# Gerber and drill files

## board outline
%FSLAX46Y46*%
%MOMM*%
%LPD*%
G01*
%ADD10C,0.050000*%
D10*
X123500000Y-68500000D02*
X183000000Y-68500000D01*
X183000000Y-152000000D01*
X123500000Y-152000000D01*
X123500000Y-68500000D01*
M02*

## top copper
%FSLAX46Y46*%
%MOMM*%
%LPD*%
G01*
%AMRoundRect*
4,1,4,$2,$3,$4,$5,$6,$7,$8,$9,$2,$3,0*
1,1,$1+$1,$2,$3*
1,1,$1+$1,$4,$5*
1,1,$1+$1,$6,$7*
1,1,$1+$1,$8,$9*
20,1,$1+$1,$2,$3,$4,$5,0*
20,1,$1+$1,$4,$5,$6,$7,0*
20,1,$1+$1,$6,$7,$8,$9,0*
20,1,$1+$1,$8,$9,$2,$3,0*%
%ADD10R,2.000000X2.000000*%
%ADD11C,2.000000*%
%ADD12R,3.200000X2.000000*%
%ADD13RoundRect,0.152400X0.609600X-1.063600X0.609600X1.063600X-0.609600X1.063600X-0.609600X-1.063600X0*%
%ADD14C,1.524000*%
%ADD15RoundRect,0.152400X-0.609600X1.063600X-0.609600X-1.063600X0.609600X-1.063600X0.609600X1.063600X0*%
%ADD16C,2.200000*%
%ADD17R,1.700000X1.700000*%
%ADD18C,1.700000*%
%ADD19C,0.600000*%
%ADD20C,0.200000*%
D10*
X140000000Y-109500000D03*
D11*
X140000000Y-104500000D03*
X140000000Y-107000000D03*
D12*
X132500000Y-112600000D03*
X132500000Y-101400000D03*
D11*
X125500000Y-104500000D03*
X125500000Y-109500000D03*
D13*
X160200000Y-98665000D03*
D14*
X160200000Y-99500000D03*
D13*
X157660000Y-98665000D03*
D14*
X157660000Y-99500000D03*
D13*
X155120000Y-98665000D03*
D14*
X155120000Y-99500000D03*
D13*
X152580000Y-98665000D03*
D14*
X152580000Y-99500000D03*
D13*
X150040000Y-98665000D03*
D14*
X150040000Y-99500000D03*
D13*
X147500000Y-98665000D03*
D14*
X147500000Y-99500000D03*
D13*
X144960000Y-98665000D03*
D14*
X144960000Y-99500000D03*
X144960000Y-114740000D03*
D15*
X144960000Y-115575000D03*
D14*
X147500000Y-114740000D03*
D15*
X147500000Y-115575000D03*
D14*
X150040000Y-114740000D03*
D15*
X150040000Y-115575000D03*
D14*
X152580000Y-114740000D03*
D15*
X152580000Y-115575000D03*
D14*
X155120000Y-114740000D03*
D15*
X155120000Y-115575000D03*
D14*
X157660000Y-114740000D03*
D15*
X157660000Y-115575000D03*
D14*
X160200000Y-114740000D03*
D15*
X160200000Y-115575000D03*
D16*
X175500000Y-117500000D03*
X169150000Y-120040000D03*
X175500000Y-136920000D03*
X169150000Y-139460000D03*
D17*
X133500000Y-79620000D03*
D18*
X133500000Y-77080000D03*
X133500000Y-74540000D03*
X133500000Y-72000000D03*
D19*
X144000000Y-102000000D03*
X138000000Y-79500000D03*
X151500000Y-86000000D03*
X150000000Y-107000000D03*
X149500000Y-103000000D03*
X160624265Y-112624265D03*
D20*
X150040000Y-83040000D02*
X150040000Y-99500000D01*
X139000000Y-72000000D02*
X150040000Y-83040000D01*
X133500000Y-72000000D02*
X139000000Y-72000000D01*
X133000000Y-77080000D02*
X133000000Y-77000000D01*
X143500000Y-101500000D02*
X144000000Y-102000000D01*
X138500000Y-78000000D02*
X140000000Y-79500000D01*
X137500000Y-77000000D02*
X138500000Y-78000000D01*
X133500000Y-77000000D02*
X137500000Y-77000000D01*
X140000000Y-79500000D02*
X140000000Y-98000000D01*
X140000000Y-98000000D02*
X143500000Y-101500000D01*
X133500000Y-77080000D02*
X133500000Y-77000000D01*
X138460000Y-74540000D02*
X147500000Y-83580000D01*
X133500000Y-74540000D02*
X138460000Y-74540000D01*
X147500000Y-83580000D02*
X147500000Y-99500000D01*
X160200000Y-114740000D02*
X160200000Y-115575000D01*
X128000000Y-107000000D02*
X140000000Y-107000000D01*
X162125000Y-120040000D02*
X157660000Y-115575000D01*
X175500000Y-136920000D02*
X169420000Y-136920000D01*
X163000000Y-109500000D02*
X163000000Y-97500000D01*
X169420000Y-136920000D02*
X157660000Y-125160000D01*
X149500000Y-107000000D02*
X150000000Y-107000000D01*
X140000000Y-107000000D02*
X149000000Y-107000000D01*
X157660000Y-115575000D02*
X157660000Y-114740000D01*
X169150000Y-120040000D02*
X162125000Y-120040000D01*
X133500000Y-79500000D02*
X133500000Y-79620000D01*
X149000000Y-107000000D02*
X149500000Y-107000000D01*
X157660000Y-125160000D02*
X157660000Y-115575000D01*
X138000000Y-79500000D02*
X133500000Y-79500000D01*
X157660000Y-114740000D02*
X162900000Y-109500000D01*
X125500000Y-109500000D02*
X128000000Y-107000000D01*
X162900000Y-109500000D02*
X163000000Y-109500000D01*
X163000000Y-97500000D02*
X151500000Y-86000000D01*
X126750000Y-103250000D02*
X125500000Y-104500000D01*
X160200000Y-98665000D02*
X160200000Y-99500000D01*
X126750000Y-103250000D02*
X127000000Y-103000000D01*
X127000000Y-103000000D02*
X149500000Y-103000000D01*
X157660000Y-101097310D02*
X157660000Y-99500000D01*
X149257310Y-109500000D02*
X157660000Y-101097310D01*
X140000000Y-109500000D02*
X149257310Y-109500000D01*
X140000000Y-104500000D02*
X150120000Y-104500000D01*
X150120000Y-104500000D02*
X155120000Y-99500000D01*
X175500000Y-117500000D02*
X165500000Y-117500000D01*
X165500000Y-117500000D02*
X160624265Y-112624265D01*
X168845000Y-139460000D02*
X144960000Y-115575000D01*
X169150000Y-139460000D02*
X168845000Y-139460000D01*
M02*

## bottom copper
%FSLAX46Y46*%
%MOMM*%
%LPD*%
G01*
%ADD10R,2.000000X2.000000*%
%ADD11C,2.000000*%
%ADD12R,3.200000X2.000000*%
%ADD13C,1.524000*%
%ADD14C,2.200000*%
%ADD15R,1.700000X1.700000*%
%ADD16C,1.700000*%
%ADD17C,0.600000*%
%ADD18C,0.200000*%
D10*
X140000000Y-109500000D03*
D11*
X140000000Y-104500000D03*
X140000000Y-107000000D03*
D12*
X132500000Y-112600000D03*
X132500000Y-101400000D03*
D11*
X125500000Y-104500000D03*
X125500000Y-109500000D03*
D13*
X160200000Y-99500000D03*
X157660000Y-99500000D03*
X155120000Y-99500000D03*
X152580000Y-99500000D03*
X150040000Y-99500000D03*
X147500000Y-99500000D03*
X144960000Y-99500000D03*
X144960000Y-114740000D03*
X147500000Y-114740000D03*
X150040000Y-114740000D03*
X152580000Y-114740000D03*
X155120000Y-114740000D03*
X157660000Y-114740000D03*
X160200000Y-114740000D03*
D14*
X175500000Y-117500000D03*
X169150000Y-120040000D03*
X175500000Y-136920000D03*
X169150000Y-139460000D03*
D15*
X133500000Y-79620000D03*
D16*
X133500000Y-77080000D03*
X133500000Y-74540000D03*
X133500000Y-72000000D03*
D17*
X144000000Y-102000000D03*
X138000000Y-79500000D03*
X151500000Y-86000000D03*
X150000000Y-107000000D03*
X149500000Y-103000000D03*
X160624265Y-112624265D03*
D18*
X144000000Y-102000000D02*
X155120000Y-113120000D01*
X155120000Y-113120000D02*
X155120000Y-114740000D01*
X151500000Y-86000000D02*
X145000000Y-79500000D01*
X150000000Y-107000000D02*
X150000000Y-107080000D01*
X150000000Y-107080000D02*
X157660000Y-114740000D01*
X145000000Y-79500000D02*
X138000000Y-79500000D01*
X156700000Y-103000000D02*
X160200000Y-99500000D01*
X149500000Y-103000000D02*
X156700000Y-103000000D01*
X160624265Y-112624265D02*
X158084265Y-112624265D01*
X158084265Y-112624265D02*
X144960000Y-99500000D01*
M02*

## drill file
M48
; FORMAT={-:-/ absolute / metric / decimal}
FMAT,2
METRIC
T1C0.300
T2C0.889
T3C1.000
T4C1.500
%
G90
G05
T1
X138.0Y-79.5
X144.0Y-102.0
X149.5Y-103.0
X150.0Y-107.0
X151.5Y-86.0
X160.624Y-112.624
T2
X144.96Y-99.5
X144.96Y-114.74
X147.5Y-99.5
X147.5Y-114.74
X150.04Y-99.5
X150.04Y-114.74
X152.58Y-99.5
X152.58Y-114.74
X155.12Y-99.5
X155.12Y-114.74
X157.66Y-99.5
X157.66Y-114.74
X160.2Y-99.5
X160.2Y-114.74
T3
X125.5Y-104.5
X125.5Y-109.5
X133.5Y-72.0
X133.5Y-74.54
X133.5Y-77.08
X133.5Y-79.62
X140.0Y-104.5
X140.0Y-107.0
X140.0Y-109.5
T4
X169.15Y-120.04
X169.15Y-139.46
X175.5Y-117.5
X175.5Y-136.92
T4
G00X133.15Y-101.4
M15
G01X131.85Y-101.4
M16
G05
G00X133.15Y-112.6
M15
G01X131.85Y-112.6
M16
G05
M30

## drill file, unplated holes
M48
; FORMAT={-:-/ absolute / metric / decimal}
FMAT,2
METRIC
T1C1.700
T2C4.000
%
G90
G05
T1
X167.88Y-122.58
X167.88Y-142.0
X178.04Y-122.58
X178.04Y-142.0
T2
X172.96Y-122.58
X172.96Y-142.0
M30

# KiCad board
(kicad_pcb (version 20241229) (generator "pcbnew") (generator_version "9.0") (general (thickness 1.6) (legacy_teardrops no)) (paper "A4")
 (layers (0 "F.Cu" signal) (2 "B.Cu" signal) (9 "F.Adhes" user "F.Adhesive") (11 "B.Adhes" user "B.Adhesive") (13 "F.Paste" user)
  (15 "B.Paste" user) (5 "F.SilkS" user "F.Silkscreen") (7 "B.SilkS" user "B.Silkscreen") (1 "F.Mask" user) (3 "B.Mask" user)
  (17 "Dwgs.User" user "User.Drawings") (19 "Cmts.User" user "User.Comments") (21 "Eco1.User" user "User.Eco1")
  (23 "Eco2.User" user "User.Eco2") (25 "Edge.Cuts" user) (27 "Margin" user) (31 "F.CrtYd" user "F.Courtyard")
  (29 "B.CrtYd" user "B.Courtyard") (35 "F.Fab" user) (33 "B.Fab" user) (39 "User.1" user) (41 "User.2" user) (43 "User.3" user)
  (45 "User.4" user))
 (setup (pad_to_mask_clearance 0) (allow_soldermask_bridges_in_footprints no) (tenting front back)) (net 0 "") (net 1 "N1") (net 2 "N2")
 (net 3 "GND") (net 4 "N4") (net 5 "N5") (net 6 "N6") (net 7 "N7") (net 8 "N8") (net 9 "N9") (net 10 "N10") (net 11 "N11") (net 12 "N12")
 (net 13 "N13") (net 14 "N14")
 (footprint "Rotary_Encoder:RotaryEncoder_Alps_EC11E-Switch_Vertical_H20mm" (layer "F.Cu") (at 140 109.5 180)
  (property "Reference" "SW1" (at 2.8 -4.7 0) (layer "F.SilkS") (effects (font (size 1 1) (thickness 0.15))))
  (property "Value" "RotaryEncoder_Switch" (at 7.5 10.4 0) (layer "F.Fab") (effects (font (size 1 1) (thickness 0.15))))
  (pad "A" thru_hole rect (at 0 0 180) (size 2 2) (drill 1) (layers "*.Cu" "*.Mask") (remove_unused_layers no) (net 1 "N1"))
  (pad "B" thru_hole circle (at 0 5 180) (size 2 2) (drill 1) (layers "*.Cu" "*.Mask") (remove_unused_layers no) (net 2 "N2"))
  (pad "C" thru_hole circle (at 0 2.5 180) (size 2 2) (drill 1) (layers "*.Cu" "*.Mask") (remove_unused_layers no) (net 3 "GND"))
  (pad "MP" thru_hole rect (at 7.5 -3.1 180) (size 3.2 2) (drill oval 2.8 1.5) (layers "*.Cu" "*.Mask") (remove_unused_layers no))
  (pad "MP" thru_hole rect (at 7.5 8.1 180) (size 3.2 2) (drill oval 2.8 1.5) (layers "*.Cu" "*.Mask") (remove_unused_layers no))
  (pad "S1" thru_hole circle (at 14.5 5 180) (size 2 2) (drill 1) (layers "*.Cu" "*.Mask") (remove_unused_layers no) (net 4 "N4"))
  (pad "S2" thru_hole circle (at 14.5 0 180) (size 2 2) (drill 1) (layers "*.Cu" "*.Mask") (remove_unused_layers no) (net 3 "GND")))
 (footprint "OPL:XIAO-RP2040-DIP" (layer "F.Cu") (at 152.58 107.12 -90)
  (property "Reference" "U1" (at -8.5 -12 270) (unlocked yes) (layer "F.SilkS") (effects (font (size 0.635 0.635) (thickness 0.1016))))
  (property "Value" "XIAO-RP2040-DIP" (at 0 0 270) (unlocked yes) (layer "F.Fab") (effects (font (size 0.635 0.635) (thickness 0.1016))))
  (pad "1" smd roundrect (at -8.455 -7.62 90) (size 2.432 1.524) (layers "F.Cu" "F.Mask") (roundrect_rratio 0.1) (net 4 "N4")
   (thermal_bridge_angle 45))
  (pad "1" thru_hole circle (at -7.62 -7.62 90) (size 1.524 1.524) (drill 0.889) (layers "*.Cu" "*.Mask") (remove_unused_layers no)
   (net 4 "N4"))
  (pad "2" smd roundrect (at -8.455 -5.08 90) (size 2.432 1.524) (layers "F.Cu" "F.Mask") (roundrect_rratio 0.1) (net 1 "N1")
   (thermal_bridge_angle 45))
  (pad "2" thru_hole circle (at -7.62 -5.08 90) (size 1.524 1.524) (drill 0.889) (layers "*.Cu" "*.Mask") (remove_unused_layers no)
   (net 1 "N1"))
  (pad "3" smd roundrect (at -8.455 -2.54 90) (size 2.432 1.524) (layers "F.Cu" "F.Mask") (roundrect_rratio 0.1) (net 2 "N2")
   (thermal_bridge_angle 45))
  (pad "3" thru_hole circle (at -7.62 -2.54 90) (size 1.524 1.524) (drill 0.889) (layers "*.Cu" "*.Mask") (remove_unused_layers no)
   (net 2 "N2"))
  (pad "4" smd roundrect (at -8.455 0 90) (size 2.432 1.524) (layers "F.Cu" "F.Mask") (roundrect_rratio 0.1) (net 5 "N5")
   (thermal_bridge_angle 45))
  (pad "4" thru_hole circle (at -7.62 0 90) (size 1.524 1.524) (drill 0.889) (layers "*.Cu" "*.Mask") (remove_unused_layers no) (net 5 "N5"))
  (pad "5" smd roundrect (at -8.455 2.54 90) (size 2.432 1.524) (layers "F.Cu" "F.Mask") (roundrect_rratio 0.1) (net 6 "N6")
   (thermal_bridge_angle 45))
  (pad "5" thru_hole circle (at -7.62 2.54 90) (size 1.524 1.524) (drill 0.889) (layers "*.Cu" "*.Mask") (remove_unused_layers no)
   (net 6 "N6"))
  (pad "6" smd roundrect (at -8.455 5.08 90) (size 2.432 1.524) (layers "F.Cu" "F.Mask") (roundrect_rratio 0.1) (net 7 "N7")
   (thermal_bridge_angle 45))
  (pad "6" thru_hole circle (at -7.62 5.08 90) (size 1.524 1.524) (drill 0.889) (layers "*.Cu" "*.Mask") (remove_unused_layers no)
   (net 7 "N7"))
  (pad "7" smd roundrect (at -8.455 7.62 90) (size 2.432 1.524) (layers "F.Cu" "F.Mask") (roundrect_rratio 0.1) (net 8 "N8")
   (thermal_bridge_angle 45))
  (pad "7" thru_hole circle (at -7.62 7.62 90) (size 1.524 1.524) (drill 0.889) (layers "*.Cu" "*.Mask") (remove_unused_layers no)
   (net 8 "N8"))
  (pad "8" thru_hole circle (at 7.62 7.62 270) (size 1.524 1.524) (drill 0.889) (layers "*.Cu" "*.Mask") (remove_unused_layers no)
   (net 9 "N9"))
  (pad "8" smd roundrect (at 8.455 7.62 270) (size 2.432 1.524) (layers "F.Cu" "F.Mask") (roundrect_rratio 0.1) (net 9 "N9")
   (thermal_bridge_angle 45))
  (pad "9" thru_hole circle (at 7.62 5.08 270) (size 1.524 1.524) (drill 0.889) (layers "*.Cu" "*.Mask") (remove_unused_layers no)
   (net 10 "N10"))
  (pad "9" smd roundrect (at 8.455 5.08 270) (size 2.432 1.524) (layers "F.Cu" "F.Mask") (roundrect_rratio 0.1) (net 10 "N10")
   (thermal_bridge_angle 45))
  (pad "10" thru_hole circle (at 7.62 2.54 270) (size 1.524 1.524) (drill 0.889) (layers "*.Cu" "*.Mask") (remove_unused_layers no)
   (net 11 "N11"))
  (pad "10" smd roundrect (at 8.455 2.54 270) (size 2.432 1.524) (layers "F.Cu" "F.Mask") (roundrect_rratio 0.1) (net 11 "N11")
   (thermal_bridge_angle 45))
  (pad "11" thru_hole circle (at 7.62 0 270) (size 1.524 1.524) (drill 0.889) (layers "*.Cu" "*.Mask") (remove_unused_layers no)
   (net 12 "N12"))
  (pad "11" smd roundrect (at 8.455 0 270) (size 2.432 1.524) (layers "F.Cu" "F.Mask") (roundrect_rratio 0.1) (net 12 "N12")
   (thermal_bridge_angle 45))
  (pad "12" thru_hole circle (at 7.62 -2.54 270) (size 1.524 1.524) (drill 0.889) (layers "*.Cu" "*.Mask") (remove_unused_layers no)
   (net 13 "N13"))
  (pad "12" smd roundrect (at 8.455 -2.54 270) (size 2.432 1.524) (layers "F.Cu" "F.Mask") (roundrect_rratio 0.1) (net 13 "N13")
   (thermal_bridge_angle 45))
  (pad "13" thru_hole circle (at 7.62 -5.08 270) (size 1.524 1.524) (drill 0.889) (layers "*.Cu" "*.Mask") (remove_unused_layers no)
   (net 3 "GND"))
  (pad "13" smd roundrect (at 8.455 -5.08 270) (size 2.432 1.524) (layers "F.Cu" "F.Mask") (roundrect_rratio 0.1) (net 3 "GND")
   (thermal_bridge_angle 45))
  (pad "14" thru_hole circle (at 7.62 -7.62 270) (size 1.524 1.524) (drill 0.889) (layers "*.Cu" "*.Mask") (remove_unused_layers no)
   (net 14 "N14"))
  (pad "14" smd roundrect (at 8.455 -7.62 270) (size 2.432 1.524) (layers "F.Cu" "F.Mask") (roundrect_rratio 0.1) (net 14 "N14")
   (thermal_bridge_angle 45)))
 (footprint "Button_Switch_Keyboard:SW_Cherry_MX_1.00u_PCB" (layer "F.Cu") (at 175.5 117.5)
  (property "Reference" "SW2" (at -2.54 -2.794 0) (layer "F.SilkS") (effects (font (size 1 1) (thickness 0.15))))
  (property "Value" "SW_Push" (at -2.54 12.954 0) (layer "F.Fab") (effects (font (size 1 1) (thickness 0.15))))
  (pad "" np_thru_hole circle (at -7.62 5.08) (size 1.7 1.7) (drill 1.7) (layers "*.Cu" "*.Mask"))
  (pad "" np_thru_hole circle (at -2.54 5.08) (size 4 4) (drill 4) (layers "*.Cu" "*.Mask"))
  (pad "" np_thru_hole circle (at 2.54 5.08) (size 1.7 1.7) (drill 1.7) (layers "*.Cu" "*.Mask"))
  (pad "1" thru_hole circle (at 0 0) (size 2.2 2.2) (drill 1.5) (layers "*.Cu" "*.Mask") (remove_unused_layers no) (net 8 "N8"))
  (pad "2" thru_hole circle (at -6.35 2.54) (size 2.2 2.2) (drill 1.5) (layers "*.Cu" "*.Mask") (remove_unused_layers no) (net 3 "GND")))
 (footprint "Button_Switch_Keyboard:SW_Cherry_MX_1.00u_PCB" (layer "F.Cu") (at 175.5 136.92)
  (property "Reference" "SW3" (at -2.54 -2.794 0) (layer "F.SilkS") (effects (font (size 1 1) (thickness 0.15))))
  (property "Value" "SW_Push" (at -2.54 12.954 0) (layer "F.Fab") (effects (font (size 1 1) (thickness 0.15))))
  (pad "" np_thru_hole circle (at -7.62 5.08) (size 1.7 1.7) (drill 1.7) (layers "*.Cu" "*.Mask"))
  (pad "" np_thru_hole circle (at -2.54 5.08) (size 4 4) (drill 4) (layers "*.Cu" "*.Mask"))
  (pad "" np_thru_hole circle (at 2.54 5.08) (size 1.7 1.7) (drill 1.7) (layers "*.Cu" "*.Mask"))
  (pad "1" thru_hole circle (at 0 0) (size 2.2 2.2) (drill 1.5) (layers "*.Cu" "*.Mask") (remove_unused_layers no) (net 3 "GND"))
  (pad "2" thru_hole circle (at -6.35 2.54) (size 2.2 2.2) (drill 1.5) (layers "*.Cu" "*.Mask") (remove_unused_layers no) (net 9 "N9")))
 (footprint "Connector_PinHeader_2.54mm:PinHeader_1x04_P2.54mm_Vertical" (layer "F.Cu") (at 133.5 79.62 180)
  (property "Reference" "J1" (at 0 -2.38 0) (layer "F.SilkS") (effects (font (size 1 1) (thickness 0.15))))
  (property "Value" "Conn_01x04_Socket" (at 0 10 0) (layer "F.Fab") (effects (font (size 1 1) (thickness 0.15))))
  (pad "1" thru_hole rect (at 0 0 180) (size 1.7 1.7) (drill 1) (layers "*.Cu" "*.Mask") (remove_unused_layers no) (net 3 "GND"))
  (pad "2" thru_hole circle (at 0 2.54 180) (size 1.7 1.7) (drill 1) (layers "*.Cu" "*.Mask") (remove_unused_layers no) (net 13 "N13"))
  (pad "3" thru_hole circle (at 0 5.08 180) (size 1.7 1.7) (drill 1) (layers "*.Cu" "*.Mask") (remove_unused_layers no) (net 7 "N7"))
  (pad "4" thru_hole circle (at 0 7.62 180) (size 1.7 1.7) (drill 1) (layers "*.Cu" "*.Mask") (remove_unused_layers no) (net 6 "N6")))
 (gr_rect (start 123.5 68.5) (end 183 152) (stroke (width 0.05) (type default)) (fill no) (layer "Edge.Cuts"))
 (segment (start 150.04 83.04) (end 150.04 99.5) (width 0.2) (layer "F.Cu") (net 6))
 (segment (start 139 72) (end 150.04 83.04) (width 0.2) (layer "F.Cu") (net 6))
 (segment (start 133.5 72) (end 139 72) (width 0.2) (layer "F.Cu") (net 6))
 (segment (start 133 77.08) (end 133 77) (width 0.2) (layer "F.Cu") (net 13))
 (segment (start 143.5 101.5) (end 144 102) (width 0.2) (layer "F.Cu") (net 13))
 (segment (start 138.5 78) (end 140 79.5) (width 0.2) (layer "F.Cu") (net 13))
 (segment (start 137.5 77) (end 138.5 78) (width 0.2) (layer "F.Cu") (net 13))
 (segment (start 133.5 77) (end 137.5 77) (width 0.2) (layer "F.Cu") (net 13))
 (segment (start 140 79.5) (end 140 98) (width 0.2) (layer "F.Cu") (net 13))
 (segment (start 140 98) (end 143.5 101.5) (width 0.2) (layer "F.Cu") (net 13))
 (segment (start 133.5 77.08) (end 133.5 77) (width 0.2) (layer "F.Cu") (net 13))
 (via (at 144 102) (size 0.6) (drill 0.3) (layers "F.Cu" "B.Cu") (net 13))
 (segment (start 144 102) (end 155.12 113.12) (width 0.2) (layer "B.Cu") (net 13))
 (segment (start 155.12 113.12) (end 155.12 114.74) (width 0.2) (layer "B.Cu") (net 13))
 (segment (start 138.46 74.54) (end 147.5 83.58) (width 0.2) (layer "F.Cu") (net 7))
 (segment (start 133.5 74.54) (end 138.46 74.54) (width 0.2) (layer "F.Cu") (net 7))
 (segment (start 147.5 83.58) (end 147.5 99.5) (width 0.2) (layer "F.Cu") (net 7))
 (segment (start 160.2 114.74) (end 160.2 115.575) (width 0.2) (layer "F.Cu") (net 14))
 (segment (start 128 107) (end 140 107) (width 0.2) (layer "F.Cu") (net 3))
 (segment (start 162.125 120.04) (end 157.66 115.575) (width 0.2) (layer "F.Cu") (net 3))
 (segment (start 175.5 136.92) (end 169.42 136.92) (width 0.2) (layer "F.Cu") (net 3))
 (segment (start 163 109.5) (end 163 97.5) (width 0.2) (layer "F.Cu") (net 3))
 (segment (start 169.42 136.92) (end 157.66 125.16) (width 0.2) (layer "F.Cu") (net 3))
 (segment (start 149.5 107) (end 150 107) (width 0.2) (layer "F.Cu") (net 3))
 (segment (start 140 107) (end 149 107) (width 0.2) (layer "F.Cu") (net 3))
 (segment (start 157.66 115.575) (end 157.66 114.74) (width 0.2) (layer "F.Cu") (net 3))
 (segment (start 169.15 120.04) (end 162.125 120.04) (width 0.2) (layer "F.Cu") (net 3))
 (segment (start 133.5 79.5) (end 133.5 79.62) (width 0.2) (layer "F.Cu") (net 3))
 (segment (start 149 107) (end 149.5 107) (width 0.2) (layer "F.Cu") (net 3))
 (segment (start 157.66 125.16) (end 157.66 115.575) (width 0.2) (layer "F.Cu") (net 3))
 (segment (start 138 79.5) (end 133.5 79.5) (width 0.2) (layer "F.Cu") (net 3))
 (segment (start 157.66 114.74) (end 162.9 109.5) (width 0.2) (layer "F.Cu") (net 3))
 (segment (start 125.5 109.5) (end 128 107) (width 0.2) (layer "F.Cu") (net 3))
 (segment (start 162.9 109.5) (end 163 109.5) (width 0.2) (layer "F.Cu") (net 3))
 (segment (start 163 97.5) (end 151.5 86) (width 0.2) (layer "F.Cu") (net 3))
 (via (at 138 79.5) (size 0.6) (drill 0.3) (layers "F.Cu" "B.Cu") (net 3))
 (via (at 151.5 86) (size 0.6) (drill 0.3) (layers "F.Cu" "B.Cu") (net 3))
 (via (at 150 107) (size 0.6) (drill 0.3) (layers "F.Cu" "B.Cu") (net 3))
 (segment (start 151.5 86) (end 145 79.5) (width 0.2) (layer "B.Cu") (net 3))
 (segment (start 150 107) (end 150 107.08) (width 0.2) (layer "B.Cu") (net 3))
 (segment (start 150 107.08) (end 157.66 114.74) (width 0.2) (layer "B.Cu") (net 3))
 (segment (start 145 79.5) (end 138 79.5) (width 0.2) (layer "B.Cu") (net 3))
 (segment (start 126.75 103.25) (end 125.5 104.5) (width 0.2) (layer "F.Cu") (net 4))
 (segment (start 160.2 98.665) (end 160.2 99.5) (width 0.2) (layer "F.Cu") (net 4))
 (segment (start 126.75 103.25) (end 127 103) (width 0.2) (layer "F.Cu") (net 4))
 (segment (start 127 103) (end 149.5 103) (width 0.2) (layer "F.Cu") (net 4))
 (via (at 149.5 103) (size 0.6) (drill 0.3) (layers "F.Cu" "B.Cu") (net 4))
 (segment (start 156.7 103) (end 160.2 99.5) (width 0.2) (layer "B.Cu") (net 4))
 (segment (start 149.5 103) (end 156.7 103) (width 0.2) (layer "B.Cu") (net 4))
 (segment (start 157.66 101.09731) (end 157.66 99.5) (width 0.2) (layer "F.Cu") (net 1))
 (segment (start 149.25731 109.5) (end 157.66 101.09731) (width 0.2) (layer "F.Cu") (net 1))
 (segment (start 140 109.5) (end 149.25731 109.5) (width 0.2) (layer "F.Cu") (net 1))
 (segment (start 140 104.5) (end 150.12 104.5) (width 0.2) (layer "F.Cu") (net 2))
 (segment (start 150.12 104.5) (end 155.12 99.5) (width 0.2) (layer "F.Cu") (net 2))
 (segment (start 175.5 117.5) (end 165.5 117.5) (width 0.2) (layer "F.Cu") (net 8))
 (segment (start 165.5 117.5) (end 160.624265 112.624265) (width 0.2) (layer "F.Cu") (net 8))
 (via (at 160.624265 112.624265) (size 0.6) (drill 0.3) (layers "F.Cu" "B.Cu") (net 8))
 (segment (start 160.624265 112.624265) (end 158.084265 112.624265) (width 0.2) (layer "B.Cu") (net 8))
 (segment (start 158.084265 112.624265) (end 144.96 99.5) (width 0.2) (layer "B.Cu") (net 8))
 (segment (start 168.845 139.46) (end 144.96 115.575) (width 0.2) (layer "F.Cu") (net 9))
 (segment (start 169.15 139.46) (end 168.845 139.46) (width 0.2) (layer "F.Cu") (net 9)))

